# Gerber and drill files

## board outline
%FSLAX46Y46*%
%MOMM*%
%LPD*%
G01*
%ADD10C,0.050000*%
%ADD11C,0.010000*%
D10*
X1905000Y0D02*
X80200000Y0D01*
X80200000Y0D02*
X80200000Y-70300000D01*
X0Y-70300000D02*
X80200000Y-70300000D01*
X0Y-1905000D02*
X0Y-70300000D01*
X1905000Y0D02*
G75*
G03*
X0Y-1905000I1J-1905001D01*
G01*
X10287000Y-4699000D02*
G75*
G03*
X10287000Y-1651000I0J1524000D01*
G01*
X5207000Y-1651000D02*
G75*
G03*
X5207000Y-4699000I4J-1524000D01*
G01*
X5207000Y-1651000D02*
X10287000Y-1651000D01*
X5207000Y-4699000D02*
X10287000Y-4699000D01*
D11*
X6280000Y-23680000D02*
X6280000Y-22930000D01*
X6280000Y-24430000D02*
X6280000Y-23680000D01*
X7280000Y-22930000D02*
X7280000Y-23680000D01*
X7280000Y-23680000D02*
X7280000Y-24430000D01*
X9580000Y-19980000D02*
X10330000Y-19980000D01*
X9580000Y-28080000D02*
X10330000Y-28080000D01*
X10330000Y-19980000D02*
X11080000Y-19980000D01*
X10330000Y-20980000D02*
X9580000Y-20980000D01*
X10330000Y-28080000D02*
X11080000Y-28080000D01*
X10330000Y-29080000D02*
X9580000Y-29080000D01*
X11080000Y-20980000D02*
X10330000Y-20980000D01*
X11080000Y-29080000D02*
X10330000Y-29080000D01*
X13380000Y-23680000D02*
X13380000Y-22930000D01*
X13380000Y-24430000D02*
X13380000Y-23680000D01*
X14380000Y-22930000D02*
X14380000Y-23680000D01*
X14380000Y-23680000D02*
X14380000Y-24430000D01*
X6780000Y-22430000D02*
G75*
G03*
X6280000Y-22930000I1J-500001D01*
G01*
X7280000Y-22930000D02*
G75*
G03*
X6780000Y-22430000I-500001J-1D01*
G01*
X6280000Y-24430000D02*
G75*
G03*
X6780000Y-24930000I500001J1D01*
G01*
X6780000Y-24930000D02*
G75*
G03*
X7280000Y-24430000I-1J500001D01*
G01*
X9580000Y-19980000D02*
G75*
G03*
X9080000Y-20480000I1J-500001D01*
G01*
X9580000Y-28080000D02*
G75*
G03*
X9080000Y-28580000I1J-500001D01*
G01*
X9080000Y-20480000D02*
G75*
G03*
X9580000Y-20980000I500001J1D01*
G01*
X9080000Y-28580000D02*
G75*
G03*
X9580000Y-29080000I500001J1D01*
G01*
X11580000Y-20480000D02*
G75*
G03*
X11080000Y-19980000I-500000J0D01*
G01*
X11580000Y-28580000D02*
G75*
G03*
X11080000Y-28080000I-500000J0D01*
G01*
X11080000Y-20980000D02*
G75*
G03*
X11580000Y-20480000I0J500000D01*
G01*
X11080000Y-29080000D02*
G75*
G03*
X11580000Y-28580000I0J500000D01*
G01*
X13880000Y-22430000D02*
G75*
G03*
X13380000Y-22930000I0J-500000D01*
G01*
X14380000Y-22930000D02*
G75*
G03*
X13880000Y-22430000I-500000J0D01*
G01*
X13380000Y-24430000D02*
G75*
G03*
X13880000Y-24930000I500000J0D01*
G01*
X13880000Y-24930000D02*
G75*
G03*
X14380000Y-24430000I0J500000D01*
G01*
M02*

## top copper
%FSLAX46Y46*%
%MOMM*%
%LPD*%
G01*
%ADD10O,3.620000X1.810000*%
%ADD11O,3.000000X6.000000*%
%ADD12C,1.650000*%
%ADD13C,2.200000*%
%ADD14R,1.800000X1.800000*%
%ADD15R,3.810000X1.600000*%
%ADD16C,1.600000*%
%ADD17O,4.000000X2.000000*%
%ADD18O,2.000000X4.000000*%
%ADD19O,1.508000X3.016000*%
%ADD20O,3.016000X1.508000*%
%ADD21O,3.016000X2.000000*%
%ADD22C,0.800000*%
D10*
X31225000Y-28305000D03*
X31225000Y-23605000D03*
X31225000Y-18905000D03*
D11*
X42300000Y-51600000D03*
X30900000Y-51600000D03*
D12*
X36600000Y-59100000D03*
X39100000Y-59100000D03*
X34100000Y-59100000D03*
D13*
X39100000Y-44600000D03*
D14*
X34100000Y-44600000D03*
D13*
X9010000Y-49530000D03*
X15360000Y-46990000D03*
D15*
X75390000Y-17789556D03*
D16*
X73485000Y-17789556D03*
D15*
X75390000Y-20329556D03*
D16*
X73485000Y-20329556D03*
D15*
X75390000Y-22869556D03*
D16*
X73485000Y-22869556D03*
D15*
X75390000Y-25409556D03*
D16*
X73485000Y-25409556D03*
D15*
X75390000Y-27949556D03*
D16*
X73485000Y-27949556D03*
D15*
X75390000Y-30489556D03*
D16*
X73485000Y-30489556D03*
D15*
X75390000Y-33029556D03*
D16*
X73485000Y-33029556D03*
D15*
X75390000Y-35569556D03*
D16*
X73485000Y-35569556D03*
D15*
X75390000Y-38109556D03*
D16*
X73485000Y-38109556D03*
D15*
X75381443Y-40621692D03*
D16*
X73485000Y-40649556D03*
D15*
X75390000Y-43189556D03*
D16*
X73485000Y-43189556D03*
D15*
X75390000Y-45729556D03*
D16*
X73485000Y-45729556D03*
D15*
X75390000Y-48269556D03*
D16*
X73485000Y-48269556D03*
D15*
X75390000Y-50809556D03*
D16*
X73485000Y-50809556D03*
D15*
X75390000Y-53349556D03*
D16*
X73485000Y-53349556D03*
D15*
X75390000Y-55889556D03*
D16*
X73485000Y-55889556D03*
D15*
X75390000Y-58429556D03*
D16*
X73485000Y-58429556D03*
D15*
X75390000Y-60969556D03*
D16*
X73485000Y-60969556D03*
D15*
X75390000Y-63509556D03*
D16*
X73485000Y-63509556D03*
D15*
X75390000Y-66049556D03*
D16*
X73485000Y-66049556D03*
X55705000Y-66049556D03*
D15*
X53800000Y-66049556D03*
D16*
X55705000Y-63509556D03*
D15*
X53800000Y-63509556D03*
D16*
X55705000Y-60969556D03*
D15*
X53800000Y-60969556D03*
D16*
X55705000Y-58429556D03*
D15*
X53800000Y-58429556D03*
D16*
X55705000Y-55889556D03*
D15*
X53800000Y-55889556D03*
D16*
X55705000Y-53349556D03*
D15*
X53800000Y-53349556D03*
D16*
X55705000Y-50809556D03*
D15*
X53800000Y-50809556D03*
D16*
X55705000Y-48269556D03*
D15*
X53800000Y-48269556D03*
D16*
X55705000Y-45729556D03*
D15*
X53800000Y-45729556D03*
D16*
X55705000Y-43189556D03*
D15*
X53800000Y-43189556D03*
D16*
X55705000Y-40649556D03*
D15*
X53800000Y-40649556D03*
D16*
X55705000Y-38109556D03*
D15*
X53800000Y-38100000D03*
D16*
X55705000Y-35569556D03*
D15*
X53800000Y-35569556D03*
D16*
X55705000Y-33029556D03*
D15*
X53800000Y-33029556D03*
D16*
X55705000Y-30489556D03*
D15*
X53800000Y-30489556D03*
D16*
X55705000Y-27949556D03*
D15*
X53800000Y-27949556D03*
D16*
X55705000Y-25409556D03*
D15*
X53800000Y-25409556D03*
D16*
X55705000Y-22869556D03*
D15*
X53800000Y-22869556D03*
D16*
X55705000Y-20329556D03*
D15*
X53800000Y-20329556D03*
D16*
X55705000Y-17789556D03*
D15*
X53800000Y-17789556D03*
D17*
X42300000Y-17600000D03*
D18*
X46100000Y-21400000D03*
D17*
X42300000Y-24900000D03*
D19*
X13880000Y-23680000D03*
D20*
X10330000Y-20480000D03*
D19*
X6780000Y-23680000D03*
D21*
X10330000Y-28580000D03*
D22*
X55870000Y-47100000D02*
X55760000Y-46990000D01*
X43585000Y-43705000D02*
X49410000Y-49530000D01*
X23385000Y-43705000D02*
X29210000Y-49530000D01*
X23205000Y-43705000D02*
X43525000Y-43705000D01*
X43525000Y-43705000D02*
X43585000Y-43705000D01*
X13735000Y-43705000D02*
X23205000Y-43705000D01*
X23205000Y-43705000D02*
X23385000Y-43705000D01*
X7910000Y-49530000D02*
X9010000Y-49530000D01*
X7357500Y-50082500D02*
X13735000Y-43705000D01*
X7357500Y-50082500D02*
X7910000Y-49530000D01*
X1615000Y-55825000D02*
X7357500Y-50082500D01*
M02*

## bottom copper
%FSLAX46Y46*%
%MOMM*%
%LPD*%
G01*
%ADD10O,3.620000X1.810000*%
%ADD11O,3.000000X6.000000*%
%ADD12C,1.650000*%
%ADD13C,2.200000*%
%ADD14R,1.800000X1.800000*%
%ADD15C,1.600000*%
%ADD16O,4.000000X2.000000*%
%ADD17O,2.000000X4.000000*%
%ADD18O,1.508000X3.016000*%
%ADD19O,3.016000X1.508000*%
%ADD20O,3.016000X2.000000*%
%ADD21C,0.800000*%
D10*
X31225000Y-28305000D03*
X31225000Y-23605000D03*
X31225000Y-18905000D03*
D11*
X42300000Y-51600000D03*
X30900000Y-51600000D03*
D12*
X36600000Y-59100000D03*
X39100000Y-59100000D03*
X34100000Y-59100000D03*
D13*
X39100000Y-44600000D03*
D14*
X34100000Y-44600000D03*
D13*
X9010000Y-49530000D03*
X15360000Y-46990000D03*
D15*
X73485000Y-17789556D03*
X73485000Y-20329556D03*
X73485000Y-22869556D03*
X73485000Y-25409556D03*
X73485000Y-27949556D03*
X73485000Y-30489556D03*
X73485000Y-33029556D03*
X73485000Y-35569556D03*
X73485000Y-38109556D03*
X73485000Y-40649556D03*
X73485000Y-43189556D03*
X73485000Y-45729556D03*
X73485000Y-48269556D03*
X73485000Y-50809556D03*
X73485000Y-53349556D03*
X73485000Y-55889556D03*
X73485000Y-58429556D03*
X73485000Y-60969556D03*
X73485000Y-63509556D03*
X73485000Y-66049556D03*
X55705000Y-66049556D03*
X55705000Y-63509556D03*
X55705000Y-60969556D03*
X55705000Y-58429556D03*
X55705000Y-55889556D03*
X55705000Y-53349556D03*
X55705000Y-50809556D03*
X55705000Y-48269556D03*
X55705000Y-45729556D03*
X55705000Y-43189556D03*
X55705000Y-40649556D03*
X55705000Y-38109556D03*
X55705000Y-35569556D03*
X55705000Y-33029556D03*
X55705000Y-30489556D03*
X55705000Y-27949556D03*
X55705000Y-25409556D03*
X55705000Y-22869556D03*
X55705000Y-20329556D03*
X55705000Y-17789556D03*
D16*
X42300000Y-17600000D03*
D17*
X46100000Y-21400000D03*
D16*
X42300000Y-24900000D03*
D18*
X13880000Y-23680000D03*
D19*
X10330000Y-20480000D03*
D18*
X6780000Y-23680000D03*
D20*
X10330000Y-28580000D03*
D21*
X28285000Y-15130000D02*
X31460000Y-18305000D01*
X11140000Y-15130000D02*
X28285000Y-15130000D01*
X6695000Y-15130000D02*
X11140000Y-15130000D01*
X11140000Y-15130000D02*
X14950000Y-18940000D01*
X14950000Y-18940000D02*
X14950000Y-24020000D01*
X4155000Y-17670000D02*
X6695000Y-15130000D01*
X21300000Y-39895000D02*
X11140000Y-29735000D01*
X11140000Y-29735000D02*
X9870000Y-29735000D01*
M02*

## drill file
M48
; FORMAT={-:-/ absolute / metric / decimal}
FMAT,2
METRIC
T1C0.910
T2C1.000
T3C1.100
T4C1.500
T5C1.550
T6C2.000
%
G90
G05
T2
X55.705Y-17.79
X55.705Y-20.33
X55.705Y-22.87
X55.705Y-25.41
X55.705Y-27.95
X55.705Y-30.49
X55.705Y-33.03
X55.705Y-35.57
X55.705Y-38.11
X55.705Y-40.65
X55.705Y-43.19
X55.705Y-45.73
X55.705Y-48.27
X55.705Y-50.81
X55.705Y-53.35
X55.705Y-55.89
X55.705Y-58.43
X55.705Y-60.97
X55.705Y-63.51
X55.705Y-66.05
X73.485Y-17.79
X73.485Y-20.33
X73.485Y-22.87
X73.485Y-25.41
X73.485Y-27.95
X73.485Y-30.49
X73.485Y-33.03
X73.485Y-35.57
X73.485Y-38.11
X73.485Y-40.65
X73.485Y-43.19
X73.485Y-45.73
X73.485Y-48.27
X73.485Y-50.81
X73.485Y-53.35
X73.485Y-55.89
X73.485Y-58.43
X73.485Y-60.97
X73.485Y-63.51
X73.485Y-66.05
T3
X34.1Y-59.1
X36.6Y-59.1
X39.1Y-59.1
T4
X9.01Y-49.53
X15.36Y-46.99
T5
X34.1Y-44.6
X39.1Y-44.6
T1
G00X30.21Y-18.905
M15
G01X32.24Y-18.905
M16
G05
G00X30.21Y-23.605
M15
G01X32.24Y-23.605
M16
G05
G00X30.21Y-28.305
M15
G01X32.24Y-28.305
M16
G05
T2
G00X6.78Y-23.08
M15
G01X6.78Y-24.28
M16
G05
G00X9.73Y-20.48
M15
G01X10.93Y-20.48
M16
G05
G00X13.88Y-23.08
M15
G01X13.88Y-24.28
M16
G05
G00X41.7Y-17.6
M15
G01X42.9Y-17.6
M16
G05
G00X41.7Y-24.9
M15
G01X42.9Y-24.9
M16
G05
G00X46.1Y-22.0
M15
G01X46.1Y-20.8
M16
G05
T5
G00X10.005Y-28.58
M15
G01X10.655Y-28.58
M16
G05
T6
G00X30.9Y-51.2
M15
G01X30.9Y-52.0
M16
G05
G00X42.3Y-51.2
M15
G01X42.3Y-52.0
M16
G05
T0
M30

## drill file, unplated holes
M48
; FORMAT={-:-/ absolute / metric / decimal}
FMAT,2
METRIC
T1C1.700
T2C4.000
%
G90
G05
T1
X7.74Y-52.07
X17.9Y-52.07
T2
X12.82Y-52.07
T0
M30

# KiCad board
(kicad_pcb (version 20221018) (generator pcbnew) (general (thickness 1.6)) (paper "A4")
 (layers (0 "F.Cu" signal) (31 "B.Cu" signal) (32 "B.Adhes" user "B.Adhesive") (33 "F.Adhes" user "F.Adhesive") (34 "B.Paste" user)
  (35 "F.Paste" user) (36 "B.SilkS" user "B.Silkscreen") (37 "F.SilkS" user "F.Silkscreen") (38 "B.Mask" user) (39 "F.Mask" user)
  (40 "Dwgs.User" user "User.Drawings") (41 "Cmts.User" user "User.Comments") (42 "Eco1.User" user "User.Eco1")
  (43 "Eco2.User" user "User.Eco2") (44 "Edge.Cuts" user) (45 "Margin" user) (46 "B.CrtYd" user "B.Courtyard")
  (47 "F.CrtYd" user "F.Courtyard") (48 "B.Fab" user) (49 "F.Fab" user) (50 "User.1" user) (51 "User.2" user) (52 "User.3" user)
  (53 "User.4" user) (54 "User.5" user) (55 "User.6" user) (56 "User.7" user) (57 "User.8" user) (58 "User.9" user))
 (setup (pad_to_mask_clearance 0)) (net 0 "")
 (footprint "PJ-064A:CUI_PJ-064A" (layer "F.Cu") (at 42.3 24.9 90)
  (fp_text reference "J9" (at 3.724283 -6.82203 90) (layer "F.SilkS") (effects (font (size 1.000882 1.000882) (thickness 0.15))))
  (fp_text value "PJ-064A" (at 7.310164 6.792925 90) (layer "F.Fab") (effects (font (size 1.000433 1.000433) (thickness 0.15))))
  (pad "1" thru_hole oval (at 0 0 90) (size 2 4) (drill oval 1 2.2) (layers "*.Cu" "*.Mask") (solder_mask_margin 0.102))
  (pad "2" thru_hole oval (at 3.5 3.8 90) (size 4 2) (drill oval 2.2 1) (layers "*.Cu" "*.Mask") (solder_mask_margin 0.102))
  (pad "3" thru_hole oval (at 7.3 0 90) (size 2 4) (drill oval 1 2.2) (layers "*.Cu" "*.Mask") (solder_mask_margin 0.102)))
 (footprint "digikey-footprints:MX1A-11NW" (layer "F.Cu") (at 11.55 42.545)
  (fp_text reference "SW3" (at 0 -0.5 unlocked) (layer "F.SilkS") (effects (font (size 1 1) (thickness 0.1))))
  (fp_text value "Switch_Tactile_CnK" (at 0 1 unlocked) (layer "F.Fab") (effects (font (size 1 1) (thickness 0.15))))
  (pad "" np_thru_hole circle (at -3.81 9.525) (size 1.7 1.7) (drill 1.7) (layers "F&B.Cu" "*.Mask"))
  (pad "" np_thru_hole circle (at 1.27 9.525) (size 4 4) (drill 4) (layers "F&B.Cu" "*.Mask"))
  (pad "" np_thru_hole circle (at 6.35 9.525) (size 1.7 1.7) (drill 1.7) (layers "F&B.Cu" "*.Mask"))
  (pad "1" thru_hole circle (at 3.81 4.445) (size 2.2 2.2) (drill 1.5) (layers "*.Cu" "*.Mask"))
  (pad "2" thru_hole circle (at -2.54 6.985) (size 2.2 2.2) (drill 1.5) (layers "*.Cu" "*.Mask")))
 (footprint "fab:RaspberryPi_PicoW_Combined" (layer "F.Cu") (at 64.595 41.919556)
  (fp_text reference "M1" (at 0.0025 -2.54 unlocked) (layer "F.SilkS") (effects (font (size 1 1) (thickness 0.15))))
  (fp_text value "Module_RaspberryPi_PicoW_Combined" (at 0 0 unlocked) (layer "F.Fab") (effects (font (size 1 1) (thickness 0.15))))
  (pad "1" smd rect (at -10.795 -24.13) (size 3.81 1.6) (layers "F.Cu" "F.Paste" "F.Mask"))
  (pad "1" thru_hole circle (at -8.89 -24.13) (size 1.6 1.6) (drill 1) (layers "*.Cu" "*.Mask"))
  (pad "2" smd rect (at -10.795 -21.59) (size 3.81 1.6) (layers "F.Cu" "F.Paste" "F.Mask"))
  (pad "2" thru_hole circle (at -8.89 -21.59) (size 1.6 1.6) (drill 1) (layers "*.Cu" "*.Mask"))
  (pad "3" smd rect (at -10.795 -19.05) (size 3.81 1.6) (layers "F.Cu" "F.Paste" "F.Mask"))
  (pad "3" thru_hole circle (at -8.89 -19.05) (size 1.6 1.6) (drill 1) (layers "*.Cu" "*.Mask"))
  (pad "4" smd rect (at -10.795 -16.51) (size 3.81 1.6) (layers "F.Cu" "F.Paste" "F.Mask"))
  (pad "4" thru_hole circle (at -8.89 -16.51) (size 1.6 1.6) (drill 1) (layers "*.Cu" "*.Mask"))
  (pad "5" smd rect (at -10.795 -13.97) (size 3.81 1.6) (layers "F.Cu" "F.Paste" "F.Mask"))
  (pad "5" thru_hole circle (at -8.89 -13.97) (size 1.6 1.6) (drill 1) (layers "*.Cu" "*.Mask"))
  (pad "6" smd rect (at -10.795 -11.43) (size 3.81 1.6) (layers "F.Cu" "F.Paste" "F.Mask"))
  (pad "6" thru_hole circle (at -8.89 -11.43) (size 1.6 1.6) (drill 1) (layers "*.Cu" "*.Mask"))
  (pad "7" smd rect (at -10.795 -8.89) (size 3.81 1.6) (layers "F.Cu" "F.Paste" "F.Mask"))
  (pad "7" thru_hole circle (at -8.89 -8.89) (size 1.6 1.6) (drill 1) (layers "*.Cu" "*.Mask"))
  (pad "8" smd rect (at -10.795 -6.35) (size 3.81 1.6) (layers "F.Cu" "F.Paste" "F.Mask"))
  (pad "8" thru_hole circle (at -8.89 -6.35) (size 1.6 1.6) (drill 1) (layers "*.Cu" "*.Mask"))
  (pad "9" smd rect (at -10.795 -3.819556) (size 3.81 1.6) (layers "F.Cu" "F.Paste" "F.Mask"))
  (pad "9" thru_hole circle (at -8.89 -3.81) (size 1.6 1.6) (drill 1) (layers "*.Cu" "*.Mask"))
  (pad "10" smd rect (at -10.795 -1.27) (size 3.81 1.6) (layers "F.Cu" "F.Paste" "F.Mask"))
  (pad "10" thru_hole circle (at -8.89 -1.27) (size 1.6 1.6) (drill 1) (layers "*.Cu" "*.Mask"))
  (pad "11" smd rect (at -10.795 1.27) (size 3.81 1.6) (layers "F.Cu" "F.Paste" "F.Mask"))
  (pad "11" thru_hole circle (at -8.89 1.27) (size 1.6 1.6) (drill 1) (layers "*.Cu" "*.Mask"))
  (pad "12" smd rect (at -10.795 3.81) (size 3.81 1.6) (layers "F.Cu" "F.Paste" "F.Mask"))
  (pad "12" thru_hole circle (at -8.89 3.81) (size 1.6 1.6) (drill 1) (layers "*.Cu" "*.Mask"))
  (pad "13" smd rect (at -10.795 6.35) (size 3.81 1.6) (layers "F.Cu" "F.Paste" "F.Mask"))
  (pad "13" thru_hole circle (at -8.89 6.35) (size 1.6 1.6) (drill 1) (layers "*.Cu" "*.Mask"))
  (pad "14" smd rect (at -10.795 8.89) (size 3.81 1.6) (layers "F.Cu" "F.Paste" "F.Mask"))
  (pad "14" thru_hole circle (at -8.89 8.89) (size 1.6 1.6) (drill 1) (layers "*.Cu" "*.Mask"))
  (pad "15" smd rect (at -10.795 11.43) (size 3.81 1.6) (layers "F.Cu" "F.Paste" "F.Mask"))
  (pad "15" thru_hole circle (at -8.89 11.43) (size 1.6 1.6) (drill 1) (layers "*.Cu" "*.Mask"))
  (pad "16" smd rect (at -10.795 13.97) (size 3.81 1.6) (layers "F.Cu" "F.Paste" "F.Mask"))
  (pad "16" thru_hole circle (at -8.89 13.97) (size 1.6 1.6) (drill 1) (layers "*.Cu" "*.Mask"))
  (pad "17" smd rect (at -10.795 16.51) (size 3.81 1.6) (layers "F.Cu" "F.Paste" "F.Mask"))
  (pad "17" thru_hole circle (at -8.89 16.51) (size 1.6 1.6) (drill 1) (layers "*.Cu" "*.Mask"))
  (pad "18" smd rect (at -10.795 19.05) (size 3.81 1.6) (layers "F.Cu" "F.Paste" "F.Mask"))
  (pad "18" thru_hole circle (at -8.89 19.05) (size 1.6 1.6) (drill 1) (layers "*.Cu" "*.Mask"))
  (pad "19" smd rect (at -10.795 21.59) (size 3.81 1.6) (layers "F.Cu" "F.Paste" "F.Mask"))
  (pad "19" thru_hole circle (at -8.89 21.59) (size 1.6 1.6) (drill 1) (layers "*.Cu" "*.Mask"))
  (pad "20" smd rect (at -10.795 24.13) (size 3.81 1.6) (layers "F.Cu" "F.Paste" "F.Mask"))
  (pad "20" thru_hole circle (at -8.89 24.13) (size 1.6 1.6) (drill 1) (layers "*.Cu" "*.Mask"))
  (pad "21" thru_hole circle (at 8.89 24.13) (size 1.6 1.6) (drill 1) (layers "*.Cu" "*.Mask"))
  (pad "21" smd rect (at 10.795 24.13) (size 3.81 1.6) (layers "F.Cu" "F.Paste" "F.Mask"))
  (pad "22" thru_hole circle (at 8.89 21.59) (size 1.6 1.6) (drill 1) (layers "*.Cu" "*.Mask"))
  (pad "22" smd rect (at 10.795 21.59) (size 3.81 1.6) (layers "F.Cu" "F.Paste" "F.Mask"))
  (pad "23" thru_hole circle (at 8.89 19.05) (size 1.6 1.6) (drill 1) (layers "*.Cu" "*.Mask"))
  (pad "23" smd rect (at 10.795 19.05) (size 3.81 1.6) (layers "F.Cu" "F.Paste" "F.Mask"))
  (pad "24" thru_hole circle (at 8.89 16.51) (size 1.6 1.6) (drill 1) (layers "*.Cu" "*.Mask"))
  (pad "24" smd rect (at 10.795 16.51) (size 3.81 1.6) (layers "F.Cu" "F.Paste" "F.Mask"))
  (pad "25" thru_hole circle (at 8.89 13.97) (size 1.6 1.6) (drill 1) (layers "*.Cu" "*.Mask"))
  (pad "25" smd rect (at 10.795 13.97) (size 3.81 1.6) (layers "F.Cu" "F.Paste" "F.Mask"))
  (pad "26" thru_hole circle (at 8.89 11.43) (size 1.6 1.6) (drill 1) (layers "*.Cu" "*.Mask"))
  (pad "26" smd rect (at 10.795 11.43) (size 3.81 1.6) (layers "F.Cu" "F.Paste" "F.Mask"))
  (pad "27" thru_hole circle (at 8.89 8.89) (size 1.6 1.6) (drill 1) (layers "*.Cu" "*.Mask"))
  (pad "27" smd rect (at 10.795 8.89) (size 3.81 1.6) (layers "F.Cu" "F.Paste" "F.Mask"))
  (pad "28" thru_hole circle (at 8.89 6.35) (size 1.6 1.6) (drill 1) (layers "*.Cu" "*.Mask"))
  (pad "28" smd rect (at 10.795 6.35) (size 3.81 1.6) (layers "F.Cu" "F.Paste" "F.Mask"))
  (pad "29" thru_hole circle (at 8.89 3.81) (size 1.6 1.6) (drill 1) (layers "*.Cu" "*.Mask"))
  (pad "29" smd rect (at 10.795 3.81) (size 3.81 1.6) (layers "F.Cu" "F.Paste" "F.Mask"))
  (pad "30" thru_hole circle (at 8.89 1.27) (size 1.6 1.6) (drill 1) (layers "*.Cu" "*.Mask"))
  (pad "30" smd rect (at 10.795 1.27) (size 3.81 1.6) (layers "F.Cu" "F.Paste" "F.Mask"))
  (pad "31" thru_hole circle (at 8.89 -1.27) (size 1.6 1.6) (drill 1) (layers "*.Cu" "*.Mask"))
  (pad "31" smd rect (at 10.786443 -1.297864) (size 3.81 1.6) (layers "F.Cu" "F.Paste" "F.Mask"))
  (pad "32" thru_hole circle (at 8.89 -3.81) (size 1.6 1.6) (drill 1) (layers "*.Cu" "*.Mask"))
  (pad "32" smd rect (at 10.795 -3.81) (size 3.81 1.6) (layers "F.Cu" "F.Paste" "F.Mask"))
  (pad "33" thru_hole circle (at 8.89 -6.35) (size 1.6 1.6) (drill 1) (layers "*.Cu" "*.Mask"))
  (pad "33" smd rect (at 10.795 -6.35) (size 3.81 1.6) (layers "F.Cu" "F.Paste" "F.Mask"))
  (pad "34" thru_hole circle (at 8.89 -8.89) (size 1.6 1.6) (drill 1) (layers "*.Cu" "*.Mask"))
  (pad "34" smd rect (at 10.795 -8.89) (size 3.81 1.6) (layers "F.Cu" "F.Paste" "F.Mask"))
  (pad "35" thru_hole circle (at 8.89 -11.43) (size 1.6 1.6) (drill 1) (layers "*.Cu" "*.Mask"))
  (pad "35" smd rect (at 10.795 -11.43) (size 3.81 1.6) (layers "F.Cu" "F.Paste" "F.Mask"))
  (pad "36" thru_hole circle (at 8.89 -13.97) (size 1.6 1.6) (drill 1) (layers "*.Cu" "*.Mask"))
  (pad "36" smd rect (at 10.795 -13.97) (size 3.81 1.6) (layers "F.Cu" "F.Paste" "F.Mask"))
  (pad "37" thru_hole circle (at 8.89 -16.51) (size 1.6 1.6) (drill 1) (layers "*.Cu" "*.Mask"))
  (pad "37" smd rect (at 10.795 -16.51) (size 3.81 1.6) (layers "F.Cu" "F.Paste" "F.Mask"))
  (pad "38" thru_hole circle (at 8.89 -19.05) (size 1.6 1.6) (drill 1) (layers "*.Cu" "*.Mask"))
  (pad "38" smd rect (at 10.795 -19.05) (size 3.81 1.6) (layers "F.Cu" "F.Paste" "F.Mask"))
  (pad "39" thru_hole circle (at 8.89 -21.59) (size 1.6 1.6) (drill 1) (layers "*.Cu" "*.Mask"))
  (pad "39" smd rect (at 10.795 -21.59) (size 3.81 1.6) (layers "F.Cu" "F.Paste" "F.Mask"))
  (pad "40" thru_hole circle (at 8.89 -24.13) (size 1.6 1.6) (drill 1) (layers "*.Cu" "*.Mask"))
  (pad "40" smd rect (at 10.795 -24.13) (size 3.81 1.6) (layers "F.Cu" "F.Paste" "F.Mask")))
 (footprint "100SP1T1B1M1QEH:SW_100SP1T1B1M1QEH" (layer "F.Cu") (at 31.225 23.605 90)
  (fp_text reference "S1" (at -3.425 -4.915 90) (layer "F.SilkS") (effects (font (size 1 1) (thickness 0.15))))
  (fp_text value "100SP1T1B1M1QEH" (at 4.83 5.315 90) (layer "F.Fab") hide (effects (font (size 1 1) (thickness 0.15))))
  (pad "1" thru_hole oval (at -4.7 0 90) (size 1.81 3.62) (drill oval 0.91 2.94) (layers "*.Cu" "*.Mask") (solder_mask_margin 0.102))
  (pad "2" thru_hole oval (at 0 0 90) (size 1.81 3.62) (drill oval 0.91 2.94) (layers "*.Cu" "*.Mask") (solder_mask_margin 0.102))
  (pad "3" thru_hole oval (at 4.7 0 90) (size 1.81 3.62) (drill oval 0.91 2.94) (layers "*.Cu" "*.Mask") (solder_mask_margin 0.102)))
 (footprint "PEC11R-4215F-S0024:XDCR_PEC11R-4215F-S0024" (layer "F.Cu") (at 36.6 51.6)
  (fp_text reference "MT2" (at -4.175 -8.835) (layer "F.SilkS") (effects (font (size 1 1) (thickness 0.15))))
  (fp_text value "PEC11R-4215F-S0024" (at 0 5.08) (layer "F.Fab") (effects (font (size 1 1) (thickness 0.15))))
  (pad "1" thru_hole rect (at -2.5 -7) (size 1.8 1.8) (drill 1.55) (layers "*.Cu" "*.Mask") (solder_mask_margin 0.102))
  (pad "2" thru_hole circle (at 2.5 -7) (size 2.2 2.2) (drill 1.55) (layers "*.Cu" "*.Mask") (solder_mask_margin 0.102))
  (pad "A" thru_hole circle (at -2.5 7.5) (size 1.65 1.65) (drill 1.1) (layers "*.Cu" "*.Mask") (solder_mask_margin 0.102))
  (pad "B" thru_hole circle (at 2.5 7.5) (size 1.65 1.65) (drill 1.1) (layers "*.Cu" "*.Mask") (solder_mask_margin 0.102))
  (pad "COM" thru_hole circle (at 0 7.5) (size 1.65 1.65) (drill 1.1) (layers "*.Cu" "*.Mask") (solder_mask_margin 0.102))
  (pad "S1" thru_hole oval (at -5.7 0) (size 3 6) (drill oval 2 2.8) (layers "*.Cu" "*.Mask") (solder_mask_margin 0.102))
  (pad "S2" thru_hole oval (at 5.7 0) (size 3 6) (drill oval 2 2.8) (layers "*.Cu" "*.Mask") (solder_mask_margin 0.102)))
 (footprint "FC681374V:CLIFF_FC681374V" (layer "F.Cu") (at 10.33 24.53)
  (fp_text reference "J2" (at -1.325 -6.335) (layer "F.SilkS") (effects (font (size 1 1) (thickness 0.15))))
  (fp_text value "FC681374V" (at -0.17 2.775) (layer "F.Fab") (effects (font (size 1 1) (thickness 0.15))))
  (fp_line (start -4.05 -0.85) (end -4.05 -1.6) (stroke (width 0.01) (type solid)) (layer "Edge.Cuts"))
  (fp_line (start -4.05 -0.1) (end -4.05 -0.85) (stroke (width 0.01) (type solid)) (layer "Edge.Cuts"))
  (fp_line (start -3.05 -1.6) (end -3.05 -0.85) (stroke (width 0.01) (type solid)) (layer "Edge.Cuts"))
  (fp_line (start -3.05 -0.85) (end -3.05 -0.1) (stroke (width 0.01) (type solid)) (layer "Edge.Cuts"))
  (fp_line (start -0.75 -4.55) (end 0 -4.55) (stroke (width 0.01) (type solid)) (layer "Edge.Cuts"))
  (fp_line (start -0.75 3.55) (end 0 3.55) (stroke (width 0.01) (type solid)) (layer "Edge.Cuts"))
  (fp_line (start 0 -4.55) (end 0.75 -4.55) (stroke (width 0.01) (type solid)) (layer "Edge.Cuts"))
  (fp_line (start 0 -3.55) (end -0.75 -3.55) (stroke (width 0.01) (type solid)) (layer "Edge.Cuts"))
  (fp_line (start 0 3.55) (end 0.75 3.55) (stroke (width 0.01) (type solid)) (layer "Edge.Cuts"))
  (fp_line (start 0 4.55) (end -0.75 4.55) (stroke (width 0.01) (type solid)) (layer "Edge.Cuts"))
  (fp_line (start 0.75 -3.55) (end 0 -3.55) (stroke (width 0.01) (type solid)) (layer "Edge.Cuts"))
  (fp_line (start 0.75 4.55) (end 0 4.55) (stroke (width 0.01) (type solid)) (layer "Edge.Cuts"))
  (fp_line (start 3.05 -0.85) (end 3.05 -1.6) (stroke (width 0.01) (type solid)) (layer "Edge.Cuts"))
  (fp_line (start 3.05 -0.1) (end 3.05 -0.85) (stroke (width 0.01) (type solid)) (layer "Edge.Cuts"))
  (fp_line (start 4.05 -1.6) (end 4.05 -0.85) (stroke (width 0.01) (type solid)) (layer "Edge.Cuts"))
  (fp_line (start 4.05 -0.85) (end 4.05 -0.1) (stroke (width 0.01) (type solid)) (layer "Edge.Cuts"))
  (fp_arc (start -4.05 -1.6) (mid -3.903553 -1.953553) (end -3.55 -2.1) (stroke (width 0.01) (type solid)) (layer "Edge.Cuts"))
  (fp_arc (start -3.55 -2.1) (mid -3.196447 -1.953553) (end -3.05 -1.6) (stroke (width 0.01) (type solid)) (layer "Edge.Cuts"))
  (fp_arc (start -3.55 0.4) (mid -3.903553 0.253553) (end -4.05 -0.1) (stroke (width 0.01) (type solid)) (layer "Edge.Cuts"))
  (fp_arc (start -3.05 -0.1) (mid -3.196447 0.253553) (end -3.55 0.4) (stroke (width 0.01) (type solid)) (layer "Edge.Cuts"))
  (fp_arc (start -1.25 -4.05) (mid -1.103553 -4.403553) (end -0.75 -4.55) (stroke (width 0.01) (type solid)) (layer "Edge.Cuts"))
  (fp_arc (start -1.25 4.05) (mid -1.103553 3.696447) (end -0.75 3.55) (stroke (width 0.01) (type solid)) (layer "Edge.Cuts"))
  (fp_arc (start -0.75 -3.55) (mid -1.103553 -3.696447) (end -1.25 -4.05) (stroke (width 0.01) (type solid)) (layer "Edge.Cuts"))
  (fp_arc (start -0.75 4.55) (mid -1.103553 4.403553) (end -1.25 4.05) (stroke (width 0.01) (type solid)) (layer "Edge.Cuts"))
  (fp_arc (start 0.75 -4.55) (mid 1.103553 -4.403553) (end 1.25 -4.05) (stroke (width 0.01) (type solid)) (layer "Edge.Cuts"))
  (fp_arc (start 0.75 3.55) (mid 1.103553 3.696447) (end 1.25 4.05) (stroke (width 0.01) (type solid)) (layer "Edge.Cuts"))
  (fp_arc (start 1.25 -4.05) (mid 1.103553 -3.696447) (end 0.75 -3.55) (stroke (width 0.01) (type solid)) (layer "Edge.Cuts"))
  (fp_arc (start 1.25 4.05) (mid 1.103553 4.403553) (end 0.75 4.55) (stroke (width 0.01) (type solid)) (layer "Edge.Cuts"))
  (fp_arc (start 3.05 -1.6) (mid 3.196447 -1.953553) (end 3.55 -2.1) (stroke (width 0.01) (type solid)) (layer "Edge.Cuts"))
  (fp_arc (start 3.55 -2.1) (mid 3.903553 -1.953553) (end 4.05 -1.6) (stroke (width 0.01) (type solid)) (layer "Edge.Cuts"))
  (fp_arc (start 3.55 0.4) (mid 3.196447 0.253553) (end 3.05 -0.1) (stroke (width 0.01) (type solid)) (layer "Edge.Cuts"))
  (fp_arc (start 4.05 -0.1) (mid 3.903553 0.253553) (end 3.55 0.4) (stroke (width 0.01) (type solid)) (layer "Edge.Cuts"))
  (pad "1" thru_hole oval (at 3.55 -0.85) (size 1.508 3.016) (drill oval 1 2.2) (layers "*.Cu" "*.Mask") (solder_mask_margin 0.102))
  (pad "2" thru_hole oval (at 0 -4.05) (size 3.016 1.508) (drill oval 2.2 1) (layers "*.Cu" "*.Mask") (solder_mask_margin 0.102))
  (pad "4" thru_hole oval (at -3.55 -0.85) (size 1.508 3.016) (drill oval 1 2.2) (layers "*.Cu" "*.Mask") (solder_mask_margin 0.102))
  (pad "5" thru_hole oval (at 0 4.05) (size 3.016 2) (drill oval 2.2 1.55) (layers "*.Cu" "*.Mask") (solder_mask_margin 0.102)))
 (gr_line (start 1.905 0) (end 80.2 0) (stroke (width 0.05) (type default)) (layer "Edge.Cuts"))
 (gr_line (start 5.207 4.699) (end 10.287 4.699) (stroke (width 0.05) (type solid)) (layer "Edge.Cuts"))
 (gr_line (start 0 70.3) (end 80.2 70.3) (stroke (width 0.05) (type default)) (layer "Edge.Cuts"))
 (gr_arc (start 10.287 1.651) (mid 11.811004 3.175002) (end 10.287 4.699) (stroke (width 0.05) (type solid)) (layer "Edge.Cuts"))
 (gr_line (start 80.2 0) (end 80.2 70.3) (stroke (width 0.05) (type default)) (layer "Edge.Cuts"))
 (gr_arc (start 5.207 4.699) (mid 3.683004 3.175002) (end 5.207 1.651) (stroke (width 0.05) (type solid)) (layer "Edge.Cuts"))
 (gr_arc (start 0 1.905) (mid 0.557962 0.557962) (end 1.905 0) (stroke (width 0.05) (type solid)) (layer "Edge.Cuts"))
 (gr_line (start 0 1.905) (end 0 70.3) (stroke (width 0.05) (type default)) (layer "Edge.Cuts"))
 (gr_line (start 5.207 1.651) (end 10.287 1.651) (stroke (width 0.05) (type solid)) (layer "Edge.Cuts"))
 (segment (start 7.91 49.53) (end 9.01 49.53) (width 0.8) (layer "F.Cu") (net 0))
 (segment (start 55.87 47.1) (end 55.76 46.99) (width 0.8) (layer "F.Cu") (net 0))
 (segment (start 23.205 43.705) (end 23.385 43.705) (width 0.8) (layer "F.Cu") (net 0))
 (segment (start 1.615 55.825) (end 7.3575 50.0825) (width 0.8) (layer "F.Cu") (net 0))
 (segment (start 7.3575 50.0825) (end 7.91 49.53) (width 0.8) (layer "F.Cu") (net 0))
 (segment (start 43.525 43.705) (end 43.585 43.705) (width 0.8) (layer "F.Cu") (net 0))
 (segment (start 43.585 43.705) (end 49.41 49.53) (width 0.8) (layer "F.Cu") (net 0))
 (segment (start 23.205 43.705) (end 43.525 43.705) (width 0.8) (layer "F.Cu") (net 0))
 (segment (start 13.735 43.705) (end 23.205 43.705) (width 0.8) (layer "F.Cu") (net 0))
 (segment (start 7.3575 50.0825) (end 13.735 43.705) (width 0.8) (layer "F.Cu") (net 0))
 (segment (start 23.385 43.705) (end 29.21 49.53) (width 0.8) (layer "F.Cu") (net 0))
 (segment (start 28.285 15.13) (end 31.46 18.305) (width 0.8) (layer "B.Cu") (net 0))
 (segment (start 14.95 18.94) (end 14.95 24.02) (width 0.8) (layer "B.Cu") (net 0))
 (segment (start 21.3 39.895) (end 11.14 29.735) (width 0.8) (layer "B.Cu") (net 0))
 (segment (start 11.14 15.13) (end 28.285 15.13) (width 0.8) (layer "B.Cu") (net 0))
 (segment (start 11.14 29.735) (end 9.87 29.735) (width 0.8) (layer "B.Cu") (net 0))
 (segment (start 4.155 17.67) (end 6.695 15.13) (width 0.8) (layer "B.Cu") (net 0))
 (segment (start 6.695 15.13) (end 11.14 15.13) (width 0.8) (layer "B.Cu") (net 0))
 (segment (start 11.14 15.13) (end 14.95 18.94) (width 0.8) (layer "B.Cu") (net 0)))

